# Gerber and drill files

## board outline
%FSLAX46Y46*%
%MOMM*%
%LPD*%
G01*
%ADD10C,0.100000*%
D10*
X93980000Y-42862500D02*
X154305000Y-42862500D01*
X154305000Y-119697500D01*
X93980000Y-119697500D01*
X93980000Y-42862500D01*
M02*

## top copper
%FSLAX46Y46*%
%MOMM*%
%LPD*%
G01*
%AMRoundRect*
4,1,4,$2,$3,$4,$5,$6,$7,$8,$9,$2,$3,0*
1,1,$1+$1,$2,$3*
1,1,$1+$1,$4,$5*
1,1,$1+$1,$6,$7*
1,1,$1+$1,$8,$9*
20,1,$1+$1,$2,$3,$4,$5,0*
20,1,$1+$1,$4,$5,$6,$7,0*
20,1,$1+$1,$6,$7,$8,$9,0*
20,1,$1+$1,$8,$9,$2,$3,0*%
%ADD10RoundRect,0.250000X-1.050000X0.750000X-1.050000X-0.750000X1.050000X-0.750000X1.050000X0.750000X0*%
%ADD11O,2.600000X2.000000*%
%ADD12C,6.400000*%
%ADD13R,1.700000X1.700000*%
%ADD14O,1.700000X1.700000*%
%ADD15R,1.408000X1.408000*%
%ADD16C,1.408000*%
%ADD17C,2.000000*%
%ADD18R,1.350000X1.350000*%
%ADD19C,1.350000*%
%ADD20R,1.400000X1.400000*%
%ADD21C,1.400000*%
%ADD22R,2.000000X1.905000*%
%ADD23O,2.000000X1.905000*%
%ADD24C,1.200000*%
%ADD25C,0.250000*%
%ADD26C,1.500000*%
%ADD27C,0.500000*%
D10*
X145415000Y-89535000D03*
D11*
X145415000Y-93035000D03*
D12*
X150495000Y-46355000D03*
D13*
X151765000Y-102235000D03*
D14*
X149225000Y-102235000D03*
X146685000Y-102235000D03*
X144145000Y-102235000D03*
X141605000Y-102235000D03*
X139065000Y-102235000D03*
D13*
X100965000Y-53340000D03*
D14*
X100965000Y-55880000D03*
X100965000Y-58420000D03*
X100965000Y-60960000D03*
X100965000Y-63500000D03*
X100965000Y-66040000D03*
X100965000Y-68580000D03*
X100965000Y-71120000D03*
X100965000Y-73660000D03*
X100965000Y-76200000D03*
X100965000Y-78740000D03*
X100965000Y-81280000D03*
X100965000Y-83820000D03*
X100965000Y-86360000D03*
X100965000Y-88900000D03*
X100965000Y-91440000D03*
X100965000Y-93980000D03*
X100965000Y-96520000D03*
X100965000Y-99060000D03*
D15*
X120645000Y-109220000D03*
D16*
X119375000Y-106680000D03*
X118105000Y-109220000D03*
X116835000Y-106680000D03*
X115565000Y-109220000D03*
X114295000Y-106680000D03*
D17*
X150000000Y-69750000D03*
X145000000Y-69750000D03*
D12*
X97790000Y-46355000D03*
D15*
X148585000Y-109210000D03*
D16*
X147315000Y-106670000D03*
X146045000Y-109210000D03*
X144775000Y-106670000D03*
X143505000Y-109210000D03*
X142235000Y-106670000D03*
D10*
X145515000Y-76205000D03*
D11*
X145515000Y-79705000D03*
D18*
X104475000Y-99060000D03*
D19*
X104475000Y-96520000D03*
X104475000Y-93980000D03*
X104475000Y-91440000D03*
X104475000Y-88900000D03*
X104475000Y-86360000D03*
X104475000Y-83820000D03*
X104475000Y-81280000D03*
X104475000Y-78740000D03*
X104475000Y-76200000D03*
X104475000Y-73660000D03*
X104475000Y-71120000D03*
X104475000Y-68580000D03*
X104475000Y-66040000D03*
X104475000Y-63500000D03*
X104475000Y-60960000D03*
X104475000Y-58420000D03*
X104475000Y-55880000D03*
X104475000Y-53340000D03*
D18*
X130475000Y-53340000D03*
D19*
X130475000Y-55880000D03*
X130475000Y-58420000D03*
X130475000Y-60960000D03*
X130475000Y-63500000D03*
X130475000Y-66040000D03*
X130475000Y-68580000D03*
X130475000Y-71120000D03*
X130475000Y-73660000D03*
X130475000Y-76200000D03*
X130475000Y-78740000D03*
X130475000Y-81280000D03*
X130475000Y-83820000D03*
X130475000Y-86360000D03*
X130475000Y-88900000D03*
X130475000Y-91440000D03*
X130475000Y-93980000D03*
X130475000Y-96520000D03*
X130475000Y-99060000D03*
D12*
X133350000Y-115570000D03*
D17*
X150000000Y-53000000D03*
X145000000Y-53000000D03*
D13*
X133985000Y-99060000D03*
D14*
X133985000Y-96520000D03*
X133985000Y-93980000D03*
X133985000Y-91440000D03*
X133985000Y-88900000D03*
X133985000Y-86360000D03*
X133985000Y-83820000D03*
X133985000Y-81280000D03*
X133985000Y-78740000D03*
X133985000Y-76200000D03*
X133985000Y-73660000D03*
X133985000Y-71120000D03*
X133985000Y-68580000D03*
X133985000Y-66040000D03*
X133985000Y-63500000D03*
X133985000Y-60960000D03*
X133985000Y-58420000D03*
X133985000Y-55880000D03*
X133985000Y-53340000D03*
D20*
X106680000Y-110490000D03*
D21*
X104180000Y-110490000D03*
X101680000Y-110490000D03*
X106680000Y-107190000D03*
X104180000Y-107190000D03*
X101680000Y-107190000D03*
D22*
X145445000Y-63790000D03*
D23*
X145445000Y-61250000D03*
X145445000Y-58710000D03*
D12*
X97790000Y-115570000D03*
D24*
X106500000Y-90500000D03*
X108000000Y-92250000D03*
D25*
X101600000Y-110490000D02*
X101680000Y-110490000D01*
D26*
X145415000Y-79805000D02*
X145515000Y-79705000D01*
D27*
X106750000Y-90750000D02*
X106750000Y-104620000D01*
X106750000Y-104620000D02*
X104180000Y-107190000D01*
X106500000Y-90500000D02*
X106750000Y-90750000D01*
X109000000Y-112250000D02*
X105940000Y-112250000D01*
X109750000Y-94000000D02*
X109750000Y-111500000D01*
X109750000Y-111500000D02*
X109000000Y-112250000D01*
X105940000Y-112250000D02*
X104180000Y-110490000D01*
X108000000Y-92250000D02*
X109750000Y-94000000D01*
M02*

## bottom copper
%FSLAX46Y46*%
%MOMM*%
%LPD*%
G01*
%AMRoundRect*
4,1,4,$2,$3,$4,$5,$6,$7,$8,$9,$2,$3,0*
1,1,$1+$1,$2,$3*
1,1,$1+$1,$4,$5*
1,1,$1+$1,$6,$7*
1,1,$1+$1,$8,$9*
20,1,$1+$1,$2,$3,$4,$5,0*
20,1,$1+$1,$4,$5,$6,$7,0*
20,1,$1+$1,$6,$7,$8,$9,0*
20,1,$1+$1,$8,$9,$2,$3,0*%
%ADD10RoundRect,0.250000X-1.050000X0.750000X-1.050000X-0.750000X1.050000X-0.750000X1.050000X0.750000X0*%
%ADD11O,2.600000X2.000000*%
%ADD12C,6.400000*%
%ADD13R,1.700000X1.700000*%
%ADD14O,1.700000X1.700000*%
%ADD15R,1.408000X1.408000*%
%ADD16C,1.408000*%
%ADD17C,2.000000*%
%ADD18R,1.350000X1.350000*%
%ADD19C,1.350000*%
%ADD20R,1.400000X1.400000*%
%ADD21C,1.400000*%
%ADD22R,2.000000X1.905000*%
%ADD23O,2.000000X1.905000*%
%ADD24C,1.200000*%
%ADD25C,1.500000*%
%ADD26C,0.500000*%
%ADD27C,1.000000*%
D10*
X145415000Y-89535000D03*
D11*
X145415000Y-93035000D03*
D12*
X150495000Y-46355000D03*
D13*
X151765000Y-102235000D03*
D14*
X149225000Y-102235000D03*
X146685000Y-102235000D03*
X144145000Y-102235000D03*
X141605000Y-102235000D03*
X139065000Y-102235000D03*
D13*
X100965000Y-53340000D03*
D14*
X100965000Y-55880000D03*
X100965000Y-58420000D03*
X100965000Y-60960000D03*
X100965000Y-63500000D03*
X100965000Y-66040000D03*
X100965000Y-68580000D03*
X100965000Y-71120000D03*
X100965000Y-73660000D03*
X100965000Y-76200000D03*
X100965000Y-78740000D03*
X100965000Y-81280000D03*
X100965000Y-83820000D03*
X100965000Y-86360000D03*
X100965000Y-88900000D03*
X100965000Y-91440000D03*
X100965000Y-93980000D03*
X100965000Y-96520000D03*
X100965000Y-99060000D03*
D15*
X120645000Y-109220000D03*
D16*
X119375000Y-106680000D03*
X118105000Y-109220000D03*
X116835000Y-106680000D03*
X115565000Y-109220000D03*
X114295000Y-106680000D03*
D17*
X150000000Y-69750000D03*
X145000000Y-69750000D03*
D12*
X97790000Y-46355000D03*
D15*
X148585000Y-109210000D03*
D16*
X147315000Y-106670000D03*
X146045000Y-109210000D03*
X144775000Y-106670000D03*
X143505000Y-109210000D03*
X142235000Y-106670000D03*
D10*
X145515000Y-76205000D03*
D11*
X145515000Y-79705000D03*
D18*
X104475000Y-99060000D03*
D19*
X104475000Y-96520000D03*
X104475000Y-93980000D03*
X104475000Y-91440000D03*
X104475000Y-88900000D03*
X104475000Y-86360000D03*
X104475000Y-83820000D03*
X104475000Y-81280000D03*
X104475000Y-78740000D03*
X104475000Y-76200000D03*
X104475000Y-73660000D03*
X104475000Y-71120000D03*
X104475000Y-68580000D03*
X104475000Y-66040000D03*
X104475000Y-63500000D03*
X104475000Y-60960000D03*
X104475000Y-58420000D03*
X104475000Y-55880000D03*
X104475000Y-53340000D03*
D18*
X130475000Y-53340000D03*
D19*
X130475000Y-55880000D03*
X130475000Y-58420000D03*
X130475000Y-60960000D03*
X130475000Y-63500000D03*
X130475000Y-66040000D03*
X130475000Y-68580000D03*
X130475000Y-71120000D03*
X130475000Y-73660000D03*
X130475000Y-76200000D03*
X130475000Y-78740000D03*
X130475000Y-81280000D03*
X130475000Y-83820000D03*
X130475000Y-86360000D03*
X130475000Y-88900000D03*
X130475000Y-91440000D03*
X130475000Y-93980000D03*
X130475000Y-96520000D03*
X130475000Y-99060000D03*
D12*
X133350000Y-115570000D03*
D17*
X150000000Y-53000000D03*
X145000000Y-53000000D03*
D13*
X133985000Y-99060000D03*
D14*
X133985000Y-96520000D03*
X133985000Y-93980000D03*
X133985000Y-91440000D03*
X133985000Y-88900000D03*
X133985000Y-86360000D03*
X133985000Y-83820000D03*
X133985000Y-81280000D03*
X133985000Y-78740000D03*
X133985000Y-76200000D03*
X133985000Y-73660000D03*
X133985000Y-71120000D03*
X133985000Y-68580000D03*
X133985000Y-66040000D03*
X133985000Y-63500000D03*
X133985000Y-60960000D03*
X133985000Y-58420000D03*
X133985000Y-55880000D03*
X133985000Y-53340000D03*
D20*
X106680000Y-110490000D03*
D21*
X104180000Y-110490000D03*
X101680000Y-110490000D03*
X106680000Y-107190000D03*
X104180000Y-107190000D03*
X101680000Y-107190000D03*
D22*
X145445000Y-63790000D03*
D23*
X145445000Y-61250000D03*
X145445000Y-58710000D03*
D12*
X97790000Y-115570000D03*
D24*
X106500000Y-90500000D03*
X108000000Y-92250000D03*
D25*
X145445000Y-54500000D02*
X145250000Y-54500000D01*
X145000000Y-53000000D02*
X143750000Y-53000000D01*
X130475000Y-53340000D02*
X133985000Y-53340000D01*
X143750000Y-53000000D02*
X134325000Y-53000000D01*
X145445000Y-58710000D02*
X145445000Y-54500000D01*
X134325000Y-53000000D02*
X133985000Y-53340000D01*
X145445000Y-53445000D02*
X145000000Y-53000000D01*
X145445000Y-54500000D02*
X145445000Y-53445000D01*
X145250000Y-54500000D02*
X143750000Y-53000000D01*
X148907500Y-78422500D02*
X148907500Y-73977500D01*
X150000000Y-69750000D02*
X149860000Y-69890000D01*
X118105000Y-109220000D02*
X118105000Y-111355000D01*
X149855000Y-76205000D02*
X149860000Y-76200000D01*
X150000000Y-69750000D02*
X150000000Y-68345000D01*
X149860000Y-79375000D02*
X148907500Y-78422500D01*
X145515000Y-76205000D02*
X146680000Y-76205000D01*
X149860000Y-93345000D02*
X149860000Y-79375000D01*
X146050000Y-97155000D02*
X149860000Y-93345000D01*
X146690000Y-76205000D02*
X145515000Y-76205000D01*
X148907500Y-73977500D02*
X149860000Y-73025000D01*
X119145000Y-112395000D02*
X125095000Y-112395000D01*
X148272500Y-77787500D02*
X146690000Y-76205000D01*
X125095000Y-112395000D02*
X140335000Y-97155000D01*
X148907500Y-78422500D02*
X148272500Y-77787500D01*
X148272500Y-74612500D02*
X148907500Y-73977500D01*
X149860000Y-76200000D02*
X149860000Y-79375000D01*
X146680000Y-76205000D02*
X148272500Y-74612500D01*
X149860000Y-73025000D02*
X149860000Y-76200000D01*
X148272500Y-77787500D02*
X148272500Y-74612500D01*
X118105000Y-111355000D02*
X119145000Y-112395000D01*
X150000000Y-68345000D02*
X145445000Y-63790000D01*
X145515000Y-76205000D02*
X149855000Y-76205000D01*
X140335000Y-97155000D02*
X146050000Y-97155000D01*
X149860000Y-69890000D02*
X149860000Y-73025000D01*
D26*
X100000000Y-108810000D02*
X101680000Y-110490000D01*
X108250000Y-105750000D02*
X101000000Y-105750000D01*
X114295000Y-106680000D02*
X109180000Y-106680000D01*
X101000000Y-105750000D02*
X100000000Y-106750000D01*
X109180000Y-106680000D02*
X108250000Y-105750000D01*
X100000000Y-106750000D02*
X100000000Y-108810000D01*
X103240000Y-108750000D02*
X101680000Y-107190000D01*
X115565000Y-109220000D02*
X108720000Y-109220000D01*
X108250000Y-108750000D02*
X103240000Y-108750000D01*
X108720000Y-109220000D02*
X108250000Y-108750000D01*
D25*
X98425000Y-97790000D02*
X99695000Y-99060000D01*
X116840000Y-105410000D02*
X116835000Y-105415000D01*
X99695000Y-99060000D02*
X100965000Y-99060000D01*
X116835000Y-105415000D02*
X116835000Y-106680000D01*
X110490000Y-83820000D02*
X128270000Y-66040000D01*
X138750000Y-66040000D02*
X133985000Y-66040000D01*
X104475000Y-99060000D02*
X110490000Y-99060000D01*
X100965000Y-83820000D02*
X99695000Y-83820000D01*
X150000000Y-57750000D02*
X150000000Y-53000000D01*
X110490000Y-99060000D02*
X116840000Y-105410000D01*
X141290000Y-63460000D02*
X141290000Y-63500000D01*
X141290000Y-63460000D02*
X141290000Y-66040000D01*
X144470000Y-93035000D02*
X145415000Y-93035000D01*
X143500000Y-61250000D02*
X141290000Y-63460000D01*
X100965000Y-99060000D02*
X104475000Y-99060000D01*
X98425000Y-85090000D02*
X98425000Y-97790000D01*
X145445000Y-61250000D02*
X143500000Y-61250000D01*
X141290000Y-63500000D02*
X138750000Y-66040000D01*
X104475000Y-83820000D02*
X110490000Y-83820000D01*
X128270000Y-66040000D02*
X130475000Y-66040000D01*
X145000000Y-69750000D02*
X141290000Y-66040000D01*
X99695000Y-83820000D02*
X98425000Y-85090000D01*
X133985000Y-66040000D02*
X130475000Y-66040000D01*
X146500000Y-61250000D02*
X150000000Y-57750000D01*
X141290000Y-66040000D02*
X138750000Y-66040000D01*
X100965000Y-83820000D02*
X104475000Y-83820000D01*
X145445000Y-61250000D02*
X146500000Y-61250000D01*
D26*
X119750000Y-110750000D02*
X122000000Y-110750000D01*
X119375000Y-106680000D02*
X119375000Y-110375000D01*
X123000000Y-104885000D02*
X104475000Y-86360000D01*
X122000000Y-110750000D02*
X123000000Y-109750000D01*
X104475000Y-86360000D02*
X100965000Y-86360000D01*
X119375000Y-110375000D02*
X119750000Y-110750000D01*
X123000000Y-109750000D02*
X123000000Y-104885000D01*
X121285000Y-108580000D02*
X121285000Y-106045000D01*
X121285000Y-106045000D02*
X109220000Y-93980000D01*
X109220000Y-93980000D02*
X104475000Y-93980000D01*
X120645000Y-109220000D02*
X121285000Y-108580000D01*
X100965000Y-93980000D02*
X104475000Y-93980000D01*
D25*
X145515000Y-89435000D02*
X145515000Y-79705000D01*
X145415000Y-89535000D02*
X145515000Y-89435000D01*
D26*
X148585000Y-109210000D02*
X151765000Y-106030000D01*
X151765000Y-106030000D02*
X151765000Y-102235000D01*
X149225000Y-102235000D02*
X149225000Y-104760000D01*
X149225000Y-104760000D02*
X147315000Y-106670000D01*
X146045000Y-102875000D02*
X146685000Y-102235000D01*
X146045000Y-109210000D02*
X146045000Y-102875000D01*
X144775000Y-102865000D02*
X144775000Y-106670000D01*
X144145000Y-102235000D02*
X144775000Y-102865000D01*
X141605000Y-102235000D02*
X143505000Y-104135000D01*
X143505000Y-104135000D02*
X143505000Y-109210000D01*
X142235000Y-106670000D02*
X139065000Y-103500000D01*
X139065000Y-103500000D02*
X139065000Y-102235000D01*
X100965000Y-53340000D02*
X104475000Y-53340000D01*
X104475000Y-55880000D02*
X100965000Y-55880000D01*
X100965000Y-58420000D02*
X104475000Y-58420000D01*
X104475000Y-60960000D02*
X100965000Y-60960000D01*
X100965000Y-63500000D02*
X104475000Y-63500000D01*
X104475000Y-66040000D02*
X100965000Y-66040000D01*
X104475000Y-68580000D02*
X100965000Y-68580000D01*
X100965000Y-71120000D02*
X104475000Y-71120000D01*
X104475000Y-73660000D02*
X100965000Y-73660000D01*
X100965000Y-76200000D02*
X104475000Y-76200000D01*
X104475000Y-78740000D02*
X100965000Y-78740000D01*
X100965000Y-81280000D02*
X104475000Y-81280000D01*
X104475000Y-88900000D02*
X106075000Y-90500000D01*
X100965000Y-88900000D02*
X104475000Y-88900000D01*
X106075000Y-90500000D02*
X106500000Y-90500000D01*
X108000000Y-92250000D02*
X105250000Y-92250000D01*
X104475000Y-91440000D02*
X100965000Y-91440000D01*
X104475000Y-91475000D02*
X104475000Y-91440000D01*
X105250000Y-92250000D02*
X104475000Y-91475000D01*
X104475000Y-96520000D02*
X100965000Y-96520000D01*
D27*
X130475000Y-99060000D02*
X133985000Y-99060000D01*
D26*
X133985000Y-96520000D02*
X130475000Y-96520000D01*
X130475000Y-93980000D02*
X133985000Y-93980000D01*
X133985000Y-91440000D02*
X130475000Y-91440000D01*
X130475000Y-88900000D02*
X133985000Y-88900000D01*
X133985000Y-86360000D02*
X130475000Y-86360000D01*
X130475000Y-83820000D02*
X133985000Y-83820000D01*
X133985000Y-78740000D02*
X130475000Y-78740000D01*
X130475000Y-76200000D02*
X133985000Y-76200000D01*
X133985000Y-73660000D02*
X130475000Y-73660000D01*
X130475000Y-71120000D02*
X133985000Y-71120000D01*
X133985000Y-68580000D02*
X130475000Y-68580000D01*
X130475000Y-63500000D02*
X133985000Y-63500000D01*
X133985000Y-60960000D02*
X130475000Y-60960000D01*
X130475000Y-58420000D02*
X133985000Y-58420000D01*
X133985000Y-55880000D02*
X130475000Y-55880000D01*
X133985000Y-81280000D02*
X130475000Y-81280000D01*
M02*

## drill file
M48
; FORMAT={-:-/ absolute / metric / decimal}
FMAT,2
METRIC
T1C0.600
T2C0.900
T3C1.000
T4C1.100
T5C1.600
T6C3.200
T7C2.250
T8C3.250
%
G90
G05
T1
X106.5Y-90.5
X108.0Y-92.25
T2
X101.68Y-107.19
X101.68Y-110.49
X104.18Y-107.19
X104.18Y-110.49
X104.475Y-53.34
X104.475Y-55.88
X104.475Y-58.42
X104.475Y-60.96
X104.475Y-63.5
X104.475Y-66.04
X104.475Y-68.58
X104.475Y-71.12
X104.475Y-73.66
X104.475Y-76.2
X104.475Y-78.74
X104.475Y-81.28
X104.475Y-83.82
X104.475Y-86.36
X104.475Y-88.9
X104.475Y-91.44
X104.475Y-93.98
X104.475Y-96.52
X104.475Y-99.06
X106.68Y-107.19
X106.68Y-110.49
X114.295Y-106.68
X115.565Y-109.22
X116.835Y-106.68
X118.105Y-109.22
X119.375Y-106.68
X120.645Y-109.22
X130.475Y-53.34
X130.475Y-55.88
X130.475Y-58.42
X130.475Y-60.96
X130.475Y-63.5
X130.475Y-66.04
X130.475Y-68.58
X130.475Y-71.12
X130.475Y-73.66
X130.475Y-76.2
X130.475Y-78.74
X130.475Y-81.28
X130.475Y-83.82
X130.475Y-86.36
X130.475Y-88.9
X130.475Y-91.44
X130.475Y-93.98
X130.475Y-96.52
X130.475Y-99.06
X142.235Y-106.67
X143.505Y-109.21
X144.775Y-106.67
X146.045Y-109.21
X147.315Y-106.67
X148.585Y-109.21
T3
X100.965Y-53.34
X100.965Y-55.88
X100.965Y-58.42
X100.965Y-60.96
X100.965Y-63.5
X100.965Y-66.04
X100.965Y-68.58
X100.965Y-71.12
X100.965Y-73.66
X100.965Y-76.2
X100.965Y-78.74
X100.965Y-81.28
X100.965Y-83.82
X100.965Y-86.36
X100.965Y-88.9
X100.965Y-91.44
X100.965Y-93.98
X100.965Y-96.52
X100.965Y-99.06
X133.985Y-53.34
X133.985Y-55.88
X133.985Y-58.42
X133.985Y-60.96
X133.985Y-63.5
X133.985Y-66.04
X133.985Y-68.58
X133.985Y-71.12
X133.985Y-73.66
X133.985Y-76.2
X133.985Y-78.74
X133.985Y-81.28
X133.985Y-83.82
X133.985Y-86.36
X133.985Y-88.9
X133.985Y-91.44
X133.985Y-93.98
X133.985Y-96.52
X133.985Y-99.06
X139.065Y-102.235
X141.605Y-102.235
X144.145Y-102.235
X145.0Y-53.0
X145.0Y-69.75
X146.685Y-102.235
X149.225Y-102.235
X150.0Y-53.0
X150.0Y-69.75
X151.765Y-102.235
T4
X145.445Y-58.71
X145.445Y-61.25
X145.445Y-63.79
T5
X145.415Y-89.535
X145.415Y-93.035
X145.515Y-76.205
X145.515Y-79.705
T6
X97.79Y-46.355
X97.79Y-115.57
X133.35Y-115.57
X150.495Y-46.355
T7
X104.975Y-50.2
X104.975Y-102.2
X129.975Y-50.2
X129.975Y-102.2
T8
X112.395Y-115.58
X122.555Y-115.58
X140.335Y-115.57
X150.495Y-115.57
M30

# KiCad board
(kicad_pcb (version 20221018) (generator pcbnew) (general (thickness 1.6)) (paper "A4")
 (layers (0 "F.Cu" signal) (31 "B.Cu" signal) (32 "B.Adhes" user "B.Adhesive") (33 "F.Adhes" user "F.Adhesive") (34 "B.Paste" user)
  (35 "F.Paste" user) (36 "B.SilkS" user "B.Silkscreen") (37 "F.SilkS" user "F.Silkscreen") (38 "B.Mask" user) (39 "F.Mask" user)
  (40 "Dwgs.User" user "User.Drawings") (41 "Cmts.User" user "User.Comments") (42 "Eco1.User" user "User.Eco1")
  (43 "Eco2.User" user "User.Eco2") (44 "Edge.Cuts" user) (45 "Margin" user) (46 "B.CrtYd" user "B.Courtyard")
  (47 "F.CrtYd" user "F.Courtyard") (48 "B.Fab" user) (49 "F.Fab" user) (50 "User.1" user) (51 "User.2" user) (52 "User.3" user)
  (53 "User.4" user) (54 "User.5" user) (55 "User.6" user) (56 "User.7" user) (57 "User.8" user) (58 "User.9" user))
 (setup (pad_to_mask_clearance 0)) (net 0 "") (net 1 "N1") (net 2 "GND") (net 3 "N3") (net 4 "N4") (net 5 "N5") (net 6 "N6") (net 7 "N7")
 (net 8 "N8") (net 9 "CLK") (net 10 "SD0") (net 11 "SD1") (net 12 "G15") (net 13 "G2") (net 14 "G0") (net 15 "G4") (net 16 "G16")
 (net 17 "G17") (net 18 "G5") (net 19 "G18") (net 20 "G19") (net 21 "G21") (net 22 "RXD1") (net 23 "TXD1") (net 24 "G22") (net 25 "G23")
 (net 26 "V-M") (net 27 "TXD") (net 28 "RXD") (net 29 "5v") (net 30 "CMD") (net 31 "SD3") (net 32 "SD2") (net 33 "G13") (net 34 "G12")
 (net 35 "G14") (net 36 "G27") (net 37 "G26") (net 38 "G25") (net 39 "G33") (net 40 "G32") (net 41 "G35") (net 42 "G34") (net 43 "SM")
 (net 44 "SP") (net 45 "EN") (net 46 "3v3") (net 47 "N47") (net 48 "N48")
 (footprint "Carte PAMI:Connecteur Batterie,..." (layer "F.Cu") (at 145.415 89.535 -90)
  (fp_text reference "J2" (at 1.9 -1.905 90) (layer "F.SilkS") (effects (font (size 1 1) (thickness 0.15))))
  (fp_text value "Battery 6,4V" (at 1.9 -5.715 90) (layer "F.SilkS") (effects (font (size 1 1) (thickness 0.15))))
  (pad "1" thru_hole roundrect (at 0 0 270) (size 2 2.6) (drill 1.6) (layers "*.Cu" "*.Mask") (roundrect_rratio 0.125) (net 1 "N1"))
  (pad "2" thru_hole oval (at 3.5 0 270) (size 2 2.6) (drill 1.6) (layers "*.Cu" "*.Mask") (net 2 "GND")))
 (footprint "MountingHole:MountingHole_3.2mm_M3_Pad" (layer "F.Cu") (at 150.495 46.355)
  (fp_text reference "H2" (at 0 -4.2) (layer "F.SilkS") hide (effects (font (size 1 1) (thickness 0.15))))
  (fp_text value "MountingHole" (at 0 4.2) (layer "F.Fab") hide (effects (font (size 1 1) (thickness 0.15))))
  (pad "1" thru_hole circle (at 0 0) (size 6.4 6.4) (drill 3.2) (layers "*.Cu" "*.Mask")))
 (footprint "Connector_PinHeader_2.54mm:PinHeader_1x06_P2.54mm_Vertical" (layer "F.Cu") (at 151.765 102.235 -90)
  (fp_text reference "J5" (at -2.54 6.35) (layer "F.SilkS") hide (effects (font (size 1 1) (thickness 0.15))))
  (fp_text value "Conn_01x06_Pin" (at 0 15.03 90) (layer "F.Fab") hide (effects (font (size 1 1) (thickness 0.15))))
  (pad "1" thru_hole rect (at 0 0 270) (size 1.7 1.7) (drill 1) (layers "*.Cu" "*.Mask") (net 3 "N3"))
  (pad "2" thru_hole oval (at 0 2.54 270) (size 1.7 1.7) (drill 1) (layers "*.Cu" "*.Mask") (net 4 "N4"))
  (pad "3" thru_hole oval (at 0 5.08 270) (size 1.7 1.7) (drill 1) (layers "*.Cu" "*.Mask") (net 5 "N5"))
  (pad "4" thru_hole oval (at 0 7.62 270) (size 1.7 1.7) (drill 1) (layers "*.Cu" "*.Mask") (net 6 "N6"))
  (pad "5" thru_hole oval (at 0 10.16 270) (size 1.7 1.7) (drill 1) (layers "*.Cu" "*.Mask") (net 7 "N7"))
  (pad "6" thru_hole oval (at 0 12.7 270) (size 1.7 1.7) (drill 1) (layers "*.Cu" "*.Mask") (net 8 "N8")))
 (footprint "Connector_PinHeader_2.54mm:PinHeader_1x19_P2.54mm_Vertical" (layer "F.Cu") (at 100.965 53.34)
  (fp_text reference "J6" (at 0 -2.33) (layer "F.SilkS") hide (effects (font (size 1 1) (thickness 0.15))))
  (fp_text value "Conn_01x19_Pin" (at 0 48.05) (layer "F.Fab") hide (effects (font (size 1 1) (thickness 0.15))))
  (pad "1" thru_hole rect (at 0 0) (size 1.7 1.7) (drill 1) (layers "*.Cu" "*.Mask") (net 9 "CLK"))
  (pad "2" thru_hole oval (at 0 2.54) (size 1.7 1.7) (drill 1) (layers "*.Cu" "*.Mask") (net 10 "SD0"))
  (pad "3" thru_hole oval (at 0 5.08) (size 1.7 1.7) (drill 1) (layers "*.Cu" "*.Mask") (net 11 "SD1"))
  (pad "4" thru_hole oval (at 0 7.62) (size 1.7 1.7) (drill 1) (layers "*.Cu" "*.Mask") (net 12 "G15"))
  (pad "5" thru_hole oval (at 0 10.16) (size 1.7 1.7) (drill 1) (layers "*.Cu" "*.Mask") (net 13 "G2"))
  (pad "6" thru_hole oval (at 0 12.7) (size 1.7 1.7) (drill 1) (layers "*.Cu" "*.Mask") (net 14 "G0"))
  (pad "7" thru_hole oval (at 0 15.24) (size 1.7 1.7) (drill 1) (layers "*.Cu" "*.Mask") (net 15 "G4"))
  (pad "8" thru_hole oval (at 0 17.78) (size 1.7 1.7) (drill 1) (layers "*.Cu" "*.Mask") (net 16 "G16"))
  (pad "9" thru_hole oval (at 0 20.32) (size 1.7 1.7) (drill 1) (layers "*.Cu" "*.Mask") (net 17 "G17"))
  (pad "10" thru_hole oval (at 0 22.86) (size 1.7 1.7) (drill 1) (layers "*.Cu" "*.Mask") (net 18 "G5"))
  (pad "11" thru_hole oval (at 0 25.4) (size 1.7 1.7) (drill 1) (layers "*.Cu" "*.Mask") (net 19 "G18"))
  (pad "12" thru_hole oval (at 0 27.94) (size 1.7 1.7) (drill 1) (layers "*.Cu" "*.Mask") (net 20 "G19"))
  (pad "13" thru_hole oval (at 0 30.48) (size 1.7 1.7) (drill 1) (layers "*.Cu" "*.Mask") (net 2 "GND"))
  (pad "14" thru_hole oval (at 0 33.02) (size 1.7 1.7) (drill 1) (layers "*.Cu" "*.Mask") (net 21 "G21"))
  (pad "15" thru_hole oval (at 0 35.56) (size 1.7 1.7) (drill 1) (layers "*.Cu" "*.Mask") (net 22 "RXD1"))
  (pad "16" thru_hole oval (at 0 38.1) (size 1.7 1.7) (drill 1) (layers "*.Cu" "*.Mask") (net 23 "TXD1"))
  (pad "17" thru_hole oval (at 0 40.64) (size 1.7 1.7) (drill 1) (layers "*.Cu" "*.Mask") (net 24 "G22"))
  (pad "18" thru_hole oval (at 0 43.18) (size 1.7 1.7) (drill 1) (layers "*.Cu" "*.Mask") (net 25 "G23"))
  (pad "19" thru_hole oval (at 0 45.72) (size 1.7 1.7) (drill 1) (layers "*.Cu" "*.Mask") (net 2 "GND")))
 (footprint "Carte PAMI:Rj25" (layer "F.Cu") (at 117.475 109.22 -90)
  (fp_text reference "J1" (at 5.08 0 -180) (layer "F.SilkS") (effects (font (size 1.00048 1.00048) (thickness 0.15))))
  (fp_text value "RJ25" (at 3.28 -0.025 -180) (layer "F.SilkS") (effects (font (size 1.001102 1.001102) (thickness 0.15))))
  (pad "" np_thru_hole circle (at 6.36 -5.08 270) (size 3.25 3.25) (drill 3.25) (layers "*.Cu" "*.Mask"))
  (pad "" np_thru_hole circle (at 6.36 5.08 270) (size 3.25 3.25) (drill 3.25) (layers "*.Cu" "*.Mask"))
  (pad "1" thru_hole rect (at 0 -3.17 270) (size 1.408 1.408) (drill 0.9) (layers "*.Cu" "*.Mask") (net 24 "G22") (solder_mask_margin 0.102))
  (pad "2" thru_hole circle (at -2.54 -1.9 270) (size 1.408 1.408) (drill 0.9) (layers "*.Cu" "*.Mask") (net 21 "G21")
   (solder_mask_margin 0.102))
  (pad "3" thru_hole circle (at 0 -0.63 270) (size 1.408 1.408) (drill 0.9) (layers "*.Cu" "*.Mask") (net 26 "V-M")
   (solder_mask_margin 0.102))
  (pad "4" thru_hole circle (at -2.54 0.64 270) (size 1.408 1.408) (drill 0.9) (layers "*.Cu" "*.Mask") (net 2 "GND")
   (solder_mask_margin 0.102))
  (pad "5" thru_hole circle (at 0 1.91 270) (size 1.408 1.408) (drill 0.9) (layers "*.Cu" "*.Mask") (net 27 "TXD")
   (solder_mask_margin 0.102))
  (pad "6" thru_hole circle (at -2.54 3.18 270) (size 1.408 1.408) (drill 0.9) (layers "*.Cu" "*.Mask") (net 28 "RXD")
   (solder_mask_margin 0.102)))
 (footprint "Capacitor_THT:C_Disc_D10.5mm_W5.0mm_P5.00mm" (layer "F.Cu") (at 150 69.75 180)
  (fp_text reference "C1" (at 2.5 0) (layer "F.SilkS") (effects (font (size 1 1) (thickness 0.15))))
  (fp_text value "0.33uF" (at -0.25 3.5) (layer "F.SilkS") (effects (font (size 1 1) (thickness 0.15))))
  (pad "1" thru_hole circle (at 0 0 180) (size 2 2) (drill 1) (layers "*.Cu" "*.Mask") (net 26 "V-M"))
  (pad "2" thru_hole circle (at 5 0 180) (size 2 2) (drill 1) (layers "*.Cu" "*.Mask") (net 2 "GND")))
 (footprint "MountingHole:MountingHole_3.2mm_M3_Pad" (layer "F.Cu") (at 97.79 46.355)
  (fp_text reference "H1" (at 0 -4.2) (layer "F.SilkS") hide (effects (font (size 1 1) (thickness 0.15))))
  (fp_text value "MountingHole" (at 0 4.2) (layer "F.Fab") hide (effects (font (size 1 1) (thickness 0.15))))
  (pad "1" thru_hole circle (at 0 0) (size 6.4 6.4) (drill 3.2) (layers "*.Cu" "*.Mask")))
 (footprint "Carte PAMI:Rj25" (layer "F.Cu") (at 145.415 109.21 -90)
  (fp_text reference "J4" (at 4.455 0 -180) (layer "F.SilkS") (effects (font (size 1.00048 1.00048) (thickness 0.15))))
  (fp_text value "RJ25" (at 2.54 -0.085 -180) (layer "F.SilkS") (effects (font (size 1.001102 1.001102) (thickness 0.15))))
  (pad "" np_thru_hole circle (at 6.36 -5.08 270) (size 3.25 3.25) (drill 3.25) (layers "*.Cu" "*.Mask"))
  (pad "" np_thru_hole circle (at 6.36 5.08 270) (size 3.25 3.25) (drill 3.25) (layers "*.Cu" "*.Mask"))
  (pad "1" thru_hole rect (at 0 -3.17 270) (size 1.408 1.408) (drill 0.9) (layers "*.Cu" "*.Mask") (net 3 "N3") (solder_mask_margin 0.102))
  (pad "2" thru_hole circle (at -2.54 -1.9 270) (size 1.408 1.408) (drill 0.9) (layers "*.Cu" "*.Mask") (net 4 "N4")
   (solder_mask_margin 0.102))
  (pad "3" thru_hole circle (at 0 -0.63 270) (size 1.408 1.408) (drill 0.9) (layers "*.Cu" "*.Mask") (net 5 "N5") (solder_mask_margin 0.102))
  (pad "4" thru_hole circle (at -2.54 0.64 270) (size 1.408 1.408) (drill 0.9) (layers "*.Cu" "*.Mask") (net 6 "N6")
   (solder_mask_margin 0.102))
  (pad "5" thru_hole circle (at 0 1.91 270) (size 1.408 1.408) (drill 0.9) (layers "*.Cu" "*.Mask") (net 7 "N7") (solder_mask_margin 0.102))
  (pad "6" thru_hole circle (at -2.54 3.18 270) (size 1.408 1.408) (drill 0.9) (layers "*.Cu" "*.Mask") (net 8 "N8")
   (solder_mask_margin 0.102)))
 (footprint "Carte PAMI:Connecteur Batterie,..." (layer "F.Cu") (at 145.515 76.205 -90)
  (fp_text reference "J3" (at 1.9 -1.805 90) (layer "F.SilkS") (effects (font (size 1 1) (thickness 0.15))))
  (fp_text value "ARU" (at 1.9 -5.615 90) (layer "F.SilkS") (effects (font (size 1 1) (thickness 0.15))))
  (pad "1" thru_hole roundrect (at 0 0 270) (size 2 2.6) (drill 1.6) (layers "*.Cu" "*.Mask") (roundrect_rratio 0.125) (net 26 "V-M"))
  (pad "2" thru_hole oval (at 3.5 0 270) (size 2 2.6) (drill 1.6) (layers "*.Cu" "*.Mask") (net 1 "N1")))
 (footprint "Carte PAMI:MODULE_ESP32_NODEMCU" (layer "F.Cu") (at 117.475 76.2 180)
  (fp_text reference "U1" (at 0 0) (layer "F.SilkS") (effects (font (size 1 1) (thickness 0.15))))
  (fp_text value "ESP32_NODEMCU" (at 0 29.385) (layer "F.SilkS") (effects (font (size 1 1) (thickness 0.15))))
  (pad "" np_thru_hole circle (at -12.5 -26 180) (size 2.25 2.25) (drill 2.25) (layers "*.Cu" "*.Mask"))
  (pad "" np_thru_hole circle (at -12.5 26 180) (size 2.25 2.25) (drill 2.25) (layers "*.Cu" "*.Mask"))
  (pad "" np_thru_hole circle (at 12.5 -26 180) (size 2.25 2.25) (drill 2.25) (layers "*.Cu" "*.Mask"))
  (pad "" np_thru_hole circle (at 12.5 26 180) (size 2.25 2.25) (drill 2.25) (layers "*.Cu" "*.Mask"))
  (pad "J4_1" thru_hole rect (at 13 -22.86 180) (size 1.35 1.35) (drill 0.9) (layers "*.Cu" "*.Mask") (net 2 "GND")
   (solder_mask_margin 0.102))
  (pad "J4_2" thru_hole circle (at 13 -20.32 180) (size 1.35 1.35) (drill 0.9) (layers "*.Cu" "*.Mask") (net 25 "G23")
   (solder_mask_margin 0.102))
  (pad "J4_3" thru_hole circle (at 13 -17.78 180) (size 1.35 1.35) (drill 0.9) (layers "*.Cu" "*.Mask") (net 24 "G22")
   (solder_mask_margin 0.102))
  (pad "J4_4" thru_hole circle (at 13 -15.24 180) (size 1.35 1.35) (drill 0.9) (layers "*.Cu" "*.Mask") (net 23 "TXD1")
   (solder_mask_margin 0.102))
  (pad "J4_5" thru_hole circle (at 13 -12.7 180) (size 1.35 1.35) (drill 0.9) (layers "*.Cu" "*.Mask") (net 22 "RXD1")
   (solder_mask_margin 0.102))
  (pad "J4_6" thru_hole circle (at 13 -10.16 180) (size 1.35 1.35) (drill 0.9) (layers "*.Cu" "*.Mask") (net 21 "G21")
   (solder_mask_margin 0.102))
  (pad "J4_7" thru_hole circle (at 13 -7.62 180) (size 1.35 1.35) (drill 0.9) (layers "*.Cu" "*.Mask") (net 2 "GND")
   (solder_mask_margin 0.102))
  (pad "J4_8" thru_hole circle (at 13 -5.08 180) (size 1.35 1.35) (drill 0.9) (layers "*.Cu" "*.Mask") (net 20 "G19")
   (solder_mask_margin 0.102))
  (pad "J4_9" thru_hole circle (at 13 -2.54 180) (size 1.35 1.35) (drill 0.9) (layers "*.Cu" "*.Mask") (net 19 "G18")
   (solder_mask_margin 0.102))
  (pad "J4_10" thru_hole circle (at 13 0 180) (size 1.35 1.35) (drill 0.9) (layers "*.Cu" "*.Mask") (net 18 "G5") (solder_mask_margin 0.102))
  (pad "J4_11" thru_hole circle (at 13 2.54 180) (size 1.35 1.35) (drill 0.9) (layers "*.Cu" "*.Mask") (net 17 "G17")
   (solder_mask_margin 0.102))
  (pad "J4_12" thru_hole circle (at 13 5.08 180) (size 1.35 1.35) (drill 0.9) (layers "*.Cu" "*.Mask") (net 16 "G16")
   (solder_mask_margin 0.102))
  (pad "J4_13" thru_hole circle (at 13 7.62 180) (size 1.35 1.35) (drill 0.9) (layers "*.Cu" "*.Mask") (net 15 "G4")
   (solder_mask_margin 0.102))
  (pad "J4_14" thru_hole circle (at 13 10.16 180) (size 1.35 1.35) (drill 0.9) (layers "*.Cu" "*.Mask") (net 14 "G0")
   (solder_mask_margin 0.102))
  (pad "J4_15" thru_hole circle (at 13 12.7 180) (size 1.35 1.35) (drill 0.9) (layers "*.Cu" "*.Mask") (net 13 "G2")
   (solder_mask_margin 0.102))
  (pad "J4_16" thru_hole circle (at 13 15.24 180) (size 1.35 1.35) (drill 0.9) (layers "*.Cu" "*.Mask") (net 12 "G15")
   (solder_mask_margin 0.102))
  (pad "J4_17" thru_hole circle (at 13 17.78 180) (size 1.35 1.35) (drill 0.9) (layers "*.Cu" "*.Mask") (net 11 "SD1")
   (solder_mask_margin 0.102))
  (pad "J4_18" thru_hole circle (at 13 20.32 180) (size 1.35 1.35) (drill 0.9) (layers "*.Cu" "*.Mask") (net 10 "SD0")
   (solder_mask_margin 0.102))
  (pad "J4_19" thru_hole circle (at 13 22.86 180) (size 1.35 1.35) (drill 0.9) (layers "*.Cu" "*.Mask") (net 9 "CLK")
   (solder_mask_margin 0.102))
  (pad "J5_1" thru_hole rect (at -13 22.86 180) (size 1.35 1.35) (drill 0.9) (layers "*.Cu" "*.Mask") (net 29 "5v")
   (solder_mask_margin 0.102))
  (pad "J5_2" thru_hole circle (at -13 20.32 180) (size 1.35 1.35) (drill 0.9) (layers "*.Cu" "*.Mask") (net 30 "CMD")
   (solder_mask_margin 0.102))
  (pad "J5_3" thru_hole circle (at -13 17.78 180) (size 1.35 1.35) (drill 0.9) (layers "*.Cu" "*.Mask") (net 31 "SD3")
   (solder_mask_margin 0.102))
  (pad "J5_4" thru_hole circle (at -13 15.24 180) (size 1.35 1.35) (drill 0.9) (layers "*.Cu" "*.Mask") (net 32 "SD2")
   (solder_mask_margin 0.102))
  (pad "J5_5" thru_hole circle (at -13 12.7 180) (size 1.35 1.35) (drill 0.9) (layers "*.Cu" "*.Mask") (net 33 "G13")
   (solder_mask_margin 0.102))
  (pad "J5_6" thru_hole circle (at -13 10.16 180) (size 1.35 1.35) (drill 0.9) (layers "*.Cu" "*.Mask") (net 2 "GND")
   (solder_mask_margin 0.102))
  (pad "J5_7" thru_hole circle (at -13 7.62 180) (size 1.35 1.35) (drill 0.9) (layers "*.Cu" "*.Mask") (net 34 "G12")
   (solder_mask_margin 0.102))
  (pad "J5_8" thru_hole circle (at -13 5.08 180) (size 1.35 1.35) (drill 0.9) (layers "*.Cu" "*.Mask") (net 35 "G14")
   (solder_mask_margin 0.102))
  (pad "J5_9" thru_hole circle (at -13 2.54 180) (size 1.35 1.35) (drill 0.9) (layers "*.Cu" "*.Mask") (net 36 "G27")
   (solder_mask_margin 0.102))
  (pad "J5_10" thru_hole circle (at -13 0 180) (size 1.35 1.35) (drill 0.9) (layers "*.Cu" "*.Mask") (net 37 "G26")
   (solder_mask_margin 0.102))
  (pad "J5_11" thru_hole circle (at -13 -2.54 180) (size 1.35 1.35) (drill 0.9) (layers "*.Cu" "*.Mask") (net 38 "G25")
   (solder_mask_margin 0.102))
  (pad "J5_12" thru_hole circle (at -13 -5.08 180) (size 1.35 1.35) (drill 0.9) (layers "*.Cu" "*.Mask") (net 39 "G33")
   (solder_mask_margin 0.102))
  (pad "J5_13" thru_hole circle (at -13 -7.62 180) (size 1.35 1.35) (drill 0.9) (layers "*.Cu" "*.Mask") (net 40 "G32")
   (solder_mask_margin 0.102))
  (pad "J5_14" thru_hole circle (at -13 -10.16 180) (size 1.35 1.35) (drill 0.9) (layers "*.Cu" "*.Mask") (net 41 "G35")
   (solder_mask_margin 0.102))
  (pad "J5_15" thru_hole circle (at -13 -12.7 180) (size 1.35 1.35) (drill 0.9) (layers "*.Cu" "*.Mask") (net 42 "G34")
   (solder_mask_margin 0.102))
  (pad "J5_16" thru_hole circle (at -13 -15.24 180) (size 1.35 1.35) (drill 0.9) (layers "*.Cu" "*.Mask") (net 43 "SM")
   (solder_mask_margin 0.102))
  (pad "J5_17" thru_hole circle (at -13 -17.78 180) (size 1.35 1.35) (drill 0.9) (layers "*.Cu" "*.Mask") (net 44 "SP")
   (solder_mask_margin 0.102))
  (pad "J5_18" thru_hole circle (at -13 -20.32 180) (size 1.35 1.35) (drill 0.9) (layers "*.Cu" "*.Mask") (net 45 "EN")
   (solder_mask_margin 0.102))
  (pad "J5_19" thru_hole circle (at -13 -22.86 180) (size 1.35 1.35) (drill 0.9) (layers "*.Cu" "*.Mask") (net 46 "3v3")
   (solder_mask_margin 0.102)))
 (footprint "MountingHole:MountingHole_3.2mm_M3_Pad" (layer "F.Cu") (at 133.35 115.57)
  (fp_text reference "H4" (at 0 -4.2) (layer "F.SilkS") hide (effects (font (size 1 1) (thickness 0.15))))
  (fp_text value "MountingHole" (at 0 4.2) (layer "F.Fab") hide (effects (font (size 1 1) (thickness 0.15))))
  (pad "1" thru_hole circle (at 0 0) (size 6.4 6.4) (drill 3.2) (layers "*.Cu" "*.Mask")))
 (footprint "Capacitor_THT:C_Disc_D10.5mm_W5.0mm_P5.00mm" (layer "F.Cu") (at 150 53 180)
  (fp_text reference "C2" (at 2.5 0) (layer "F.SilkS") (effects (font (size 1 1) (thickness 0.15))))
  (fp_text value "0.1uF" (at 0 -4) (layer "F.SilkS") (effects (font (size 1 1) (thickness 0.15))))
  (pad "1" thru_hole circle (at 0 0 180) (size 2 2) (drill 1) (layers "*.Cu" "*.Mask") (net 2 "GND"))
  (pad "2" thru_hole circle (at 5 0 180) (size 2 2) (drill 1) (layers "*.Cu" "*.Mask") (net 29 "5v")))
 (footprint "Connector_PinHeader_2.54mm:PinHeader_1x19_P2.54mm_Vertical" (layer "F.Cu") (at 133.985 99.06 180)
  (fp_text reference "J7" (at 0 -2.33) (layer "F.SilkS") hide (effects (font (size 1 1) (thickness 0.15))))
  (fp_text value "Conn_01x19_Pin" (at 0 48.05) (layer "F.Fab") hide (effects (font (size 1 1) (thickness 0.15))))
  (pad "1" thru_hole rect (at 0 0 180) (size 1.7 1.7) (drill 1) (layers "*.Cu" "*.Mask") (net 46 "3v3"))
  (pad "2" thru_hole oval (at 0 2.54 180) (size 1.7 1.7) (drill 1) (layers "*.Cu" "*.Mask") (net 45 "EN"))
  (pad "3" thru_hole oval (at 0 5.08 180) (size 1.7 1.7) (drill 1) (layers "*.Cu" "*.Mask") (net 44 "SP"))
  (pad "4" thru_hole oval (at 0 7.62 180) (size 1.7 1.7) (drill 1) (layers "*.Cu" "*.Mask") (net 43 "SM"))
  (pad "5" thru_hole oval (at 0 10.16 180) (size 1.7 1.7) (drill 1) (layers "*.Cu" "*.Mask") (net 42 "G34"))
  (pad "6" thru_hole oval (at 0 12.7 180) (size 1.7 1.7) (drill 1) (layers "*.Cu" "*.Mask") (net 41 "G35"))
  (pad "7" thru_hole oval (at 0 15.24 180) (size 1.7 1.7) (drill 1) (layers "*.Cu" "*.Mask") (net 40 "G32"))
  (pad "8" thru_hole oval (at 0 17.78 180) (size 1.7 1.7) (drill 1) (layers "*.Cu" "*.Mask") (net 39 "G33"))
  (pad "9" thru_hole oval (at 0 20.32 180) (size 1.7 1.7) (drill 1) (layers "*.Cu" "*.Mask") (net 38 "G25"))
  (pad "10" thru_hole oval (at 0 22.86 180) (size 1.7 1.7) (drill 1) (layers "*.Cu" "*.Mask") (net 37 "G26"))
  (pad "11" thru_hole oval (at 0 25.4 180) (size 1.7 1.7) (drill 1) (layers "*.Cu" "*.Mask") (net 36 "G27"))
  (pad "12" thru_hole oval (at 0 27.94 180) (size 1.7 1.7) (drill 1) (layers "*.Cu" "*.Mask") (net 35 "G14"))
  (pad "13" thru_hole oval (at 0 30.48 180) (size 1.7 1.7) (drill 1) (layers "*.Cu" "*.Mask") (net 34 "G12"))
  (pad "14" thru_hole oval (at 0 33.02 180) (size 1.7 1.7) (drill 1) (layers "*.Cu" "*.Mask") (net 2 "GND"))
  (pad "15" thru_hole oval (at 0 35.56 180) (size 1.7 1.7) (drill 1) (layers "*.Cu" "*.Mask") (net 33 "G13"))
  (pad "16" thru_hole oval (at 0 38.1 180) (size 1.7 1.7) (drill 1) (layers "*.Cu" "*.Mask") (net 32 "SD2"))
  (pad "17" thru_hole oval (at 0 40.64 180) (size 1.7 1.7) (drill 1) (layers "*.Cu" "*.Mask") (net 31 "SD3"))
  (pad "18" thru_hole oval (at 0 43.18 180) (size 1.7 1.7) (drill 1) (layers "*.Cu" "*.Mask") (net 30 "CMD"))
  (pad "19" thru_hole oval (at 0 45.72 180) (size 1.7 1.7) (drill 1) (layers "*.Cu" "*.Mask") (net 29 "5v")))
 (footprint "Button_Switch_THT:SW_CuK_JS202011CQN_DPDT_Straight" (layer "F.Cu") (at 106.68 110.49 180)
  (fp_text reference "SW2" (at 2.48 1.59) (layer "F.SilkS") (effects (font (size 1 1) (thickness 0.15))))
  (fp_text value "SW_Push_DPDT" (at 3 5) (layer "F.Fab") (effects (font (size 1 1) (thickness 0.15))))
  (pad "1" thru_hole rect (at 0 0 180) (size 1.4 1.4) (drill 0.9) (layers "*.Cu" "*.Mask") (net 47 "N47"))
  (pad "2" thru_hole circle (at 2.5 0 180) (size 1.4 1.4) (drill 0.9) (layers "*.Cu" "*.Mask") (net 23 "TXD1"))
  (pad "3" thru_hole circle (at 5 0 180) (size 1.4 1.4) (drill 0.9) (layers "*.Cu" "*.Mask") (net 28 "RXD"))
  (pad "4" thru_hole circle (at 0 3.3 180) (size 1.4 1.4) (drill 0.9) (layers "*.Cu" "*.Mask") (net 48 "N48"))
  (pad "5" thru_hole circle (at 2.5 3.3 180) (size 1.4 1.4) (drill 0.9) (layers "*.Cu" "*.Mask") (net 22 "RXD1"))
  (pad "6" thru_hole circle (at 5 3.3 180) (size 1.4 1.4) (drill 0.9) (layers "*.Cu" "*.Mask") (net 27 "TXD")))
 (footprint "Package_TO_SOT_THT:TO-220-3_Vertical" (layer "F.Cu") (at 145.445 63.79 90)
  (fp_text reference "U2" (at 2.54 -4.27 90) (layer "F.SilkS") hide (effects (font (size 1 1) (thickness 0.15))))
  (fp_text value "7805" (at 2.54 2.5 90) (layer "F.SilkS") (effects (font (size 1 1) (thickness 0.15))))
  (pad "1" thru_hole rect (at 0 0 90) (size 1.905 2) (drill 1.1) (layers "*.Cu" "*.Mask") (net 26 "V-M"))
  (pad "2" thru_hole oval (at 2.54 0 90) (size 1.905 2) (drill 1.1) (layers "*.Cu" "*.Mask") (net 2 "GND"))
  (pad "3" thru_hole oval (at 5.08 0 90) (size 1.905 2) (drill 1.1) (layers "*.Cu" "*.Mask") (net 29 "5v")))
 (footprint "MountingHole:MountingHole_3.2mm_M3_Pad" (layer "F.Cu") (at 97.79 115.57)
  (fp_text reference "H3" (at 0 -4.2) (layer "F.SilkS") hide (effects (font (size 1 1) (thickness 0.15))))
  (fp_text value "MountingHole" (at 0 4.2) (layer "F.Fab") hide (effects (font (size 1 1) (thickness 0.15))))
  (pad "1" thru_hole circle (at 0 0) (size 6.4 6.4) (drill 3.2) (layers "*.Cu" "*.Mask")))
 (gr_rect (start 93.98 42.8625) (end 154.305 119.6975) (stroke (width 0.1) (type default)) (fill none) (layer "Edge.Cuts"))
 (segment (start 145.445 54.5) (end 145.25 54.5) (width 1.5) (layer "B.Cu") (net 29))
 (segment (start 145 53) (end 143.75 53) (width 1.5) (layer "B.Cu") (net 29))
 (segment (start 130.475 53.34) (end 133.985 53.34) (width 1.5) (layer "B.Cu") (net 29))
 (segment (start 143.75 53) (end 134.325 53) (width 1.5) (layer "B.Cu") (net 29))
 (segment (start 145.445 58.71) (end 145.445 54.5) (width 1.5) (layer "B.Cu") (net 29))
 (segment (start 134.325 53) (end 133.985 53.34) (width 1.5) (layer "B.Cu") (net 29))
 (segment (start 145.445 53.445) (end 145 53) (width 1.5) (layer "B.Cu") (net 29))
 (segment (start 145.445 54.5) (end 145.445 53.445) (width 1.5) (layer "B.Cu") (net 29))
 (segment (start 145.25 54.5) (end 143.75 53) (width 1.5) (layer "B.Cu") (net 29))
 (segment (start 148.9075 78.4225) (end 148.9075 73.9775) (width 1.5) (layer "B.Cu") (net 26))
 (segment (start 150 69.75) (end 149.86 69.89) (width 1.5) (layer "B.Cu") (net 26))
 (segment (start 118.105 109.22) (end 118.105 111.355) (width 1.5) (layer "B.Cu") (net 26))
 (segment (start 149.855 76.205) (end 149.86 76.2) (width 1.5) (layer "B.Cu") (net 26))
 (segment (start 150 69.75) (end 150 68.345) (width 1.5) (layer "B.Cu") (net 26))
 (segment (start 149.86 79.375) (end 148.9075 78.4225) (width 1.5) (layer "B.Cu") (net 26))
 (segment (start 145.515 76.205) (end 146.68 76.205) (width 1.5) (layer "B.Cu") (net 26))
 (segment (start 149.86 93.345) (end 149.86 79.375) (width 1.5) (layer "B.Cu") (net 26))
 (segment (start 146.05 97.155) (end 149.86 93.345) (width 1.5) (layer "B.Cu") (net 26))
 (segment (start 146.69 76.205) (end 145.515 76.205) (width 1.5) (layer "B.Cu") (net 26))
 (segment (start 148.9075 73.9775) (end 149.86 73.025) (width 1.5) (layer "B.Cu") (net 26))
 (segment (start 119.145 112.395) (end 125.095 112.395) (width 1.5) (layer "B.Cu") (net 26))
 (segment (start 148.2725 77.7875) (end 146.69 76.205) (width 1.5) (layer "B.Cu") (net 26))
 (segment (start 125.095 112.395) (end 140.335 97.155) (width 1.5) (layer "B.Cu") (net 26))
 (segment (start 148.9075 78.4225) (end 148.2725 77.7875) (width 1.5) (layer "B.Cu") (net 26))
 (segment (start 148.2725 74.6125) (end 148.9075 73.9775) (width 1.5) (layer "B.Cu") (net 26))
 (segment (start 149.86 76.2) (end 149.86 79.375) (width 1.5) (layer "B.Cu") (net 26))
 (segment (start 146.68 76.205) (end 148.2725 74.6125) (width 1.5) (layer "B.Cu") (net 26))
 (segment (start 149.86 73.025) (end 149.86 76.2) (width 1.5) (layer "B.Cu") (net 26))
 (segment (start 148.2725 77.7875) (end 148.2725 74.6125) (width 1.5) (layer "B.Cu") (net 26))
 (segment (start 118.105 111.355) (end 119.145 112.395) (width 1.5) (layer "B.Cu") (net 26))
 (segment (start 150 68.345) (end 145.445 63.79) (width 1.5) (layer "B.Cu") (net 26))
 (segment (start 145.515 76.205) (end 149.855 76.205) (width 1.5) (layer "B.Cu") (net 26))
 (segment (start 140.335 97.155) (end 146.05 97.155) (width 1.5) (layer "B.Cu") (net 26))
 (segment (start 149.86 69.89) (end 149.86 73.025) (width 1.5) (layer "B.Cu") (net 26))
 (segment (start 101.6 110.49) (end 101.68 110.49) (width 0.25) (layer "F.Cu") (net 28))
 (segment (start 100 108.81) (end 101.68 110.49) (width 0.5) (layer "B.Cu") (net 28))
 (segment (start 108.25 105.75) (end 101 105.75) (width 0.5) (layer "B.Cu") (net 28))
 (segment (start 114.295 106.68) (end 109.18 106.68) (width 0.5) (layer "B.Cu") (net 28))
 (segment (start 101 105.75) (end 100 106.75) (width 0.5) (layer "B.Cu") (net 28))
 (segment (start 109.18 106.68) (end 108.25 105.75) (width 0.5) (layer "B.Cu") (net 28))
 (segment (start 100 106.75) (end 100 108.81) (width 0.5) (layer "B.Cu") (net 28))
 (segment (start 103.24 108.75) (end 101.68 107.19) (width 0.5) (layer "B.Cu") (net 27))
 (segment (start 115.565 109.22) (end 108.72 109.22) (width 0.5) (layer "B.Cu") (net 27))
 (segment (start 108.25 108.75) (end 103.24 108.75) (width 0.5) (layer "B.Cu") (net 27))
 (segment (start 108.72 109.22) (end 108.25 108.75) (width 0.5) (layer "B.Cu") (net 27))
 (segment (start 98.425 97.79) (end 99.695 99.06) (width 1.5) (layer "B.Cu") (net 2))
 (segment (start 116.84 105.41) (end 116.835 105.415) (width 1.5) (layer "B.Cu") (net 2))
 (segment (start 99.695 99.06) (end 100.965 99.06) (width 1.5) (layer "B.Cu") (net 2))
 (segment (start 116.835 105.415) (end 116.835 106.68) (width 1.5) (layer "B.Cu") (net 2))
 (segment (start 110.49 83.82) (end 128.27 66.04) (width 1.5) (layer "B.Cu") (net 2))
 (segment (start 138.75 66.04) (end 133.985 66.04) (width 1.5) (layer "B.Cu") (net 2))
 (segment (start 104.475 99.06) (end 110.49 99.06) (width 1.5) (layer "B.Cu") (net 2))
 (segment (start 100.965 83.82) (end 99.695 83.82) (width 1.5) (layer "B.Cu") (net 2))
 (segment (start 150 57.75) (end 150 53) (width 1.5) (layer "B.Cu") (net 2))
 (segment (start 110.49 99.06) (end 116.84 105.41) (width 1.5) (layer "B.Cu") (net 2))
 (segment (start 141.29 63.46) (end 141.29 63.5) (width 1.5) (layer "B.Cu") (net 2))
 (segment (start 141.29 63.46) (end 141.29 66.04) (width 1.5) (layer "B.Cu") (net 2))
 (segment (start 144.47 93.035) (end 145.415 93.035) (width 1.5) (layer "B.Cu") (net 2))
 (segment (start 143.5 61.25) (end 141.29 63.46) (width 1.5) (layer "B.Cu") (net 2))
 (segment (start 100.965 99.06) (end 104.475 99.06) (width 1.5) (layer "B.Cu") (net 2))
 (segment (start 98.425 85.09) (end 98.425 97.79) (width 1.5) (layer "B.Cu") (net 2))
 (segment (start 145.445 61.25) (end 143.5 61.25) (width 1.5) (layer "B.Cu") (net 2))
 (segment (start 141.29 63.5) (end 138.75 66.04) (width 1.5) (layer "B.Cu") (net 2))
 (segment (start 104.475 83.82) (end 110.49 83.82) (width 1.5) (layer "B.Cu") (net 2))
 (segment (start 128.27 66.04) (end 130.475 66.04) (width 1.5) (layer "B.Cu") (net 2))
 (segment (start 145 69.75) (end 141.29 66.04) (width 1.5) (layer "B.Cu") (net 2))
 (segment (start 99.695 83.82) (end 98.425 85.09) (width 1.5) (layer "B.Cu") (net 2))
 (segment (start 133.985 66.04) (end 130.475 66.04) (width 1.5) (layer "B.Cu") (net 2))
 (segment (start 146.5 61.25) (end 150 57.75) (width 1.5) (layer "B.Cu") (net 2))
 (segment (start 141.29 66.04) (end 138.75 66.04) (width 1.5) (layer "B.Cu") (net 2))
 (segment (start 100.965 83.82) (end 104.475 83.82) (width 1.5) (layer "B.Cu") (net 2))
 (segment (start 145.445 61.25) (end 146.5 61.25) (width 1.5) (layer "B.Cu") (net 2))
 (segment (start 119.75 110.75) (end 122 110.75) (width 0.5) (layer "B.Cu") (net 21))
 (segment (start 119.375 106.68) (end 119.375 110.375) (width 0.5) (layer "B.Cu") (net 21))
 (segment (start 123 104.885) (end 104.475 86.36) (width 0.5) (layer "B.Cu") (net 21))
 (segment (start 122 110.75) (end 123 109.75) (width 0.5) (layer "B.Cu") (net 21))
 (segment (start 104.475 86.36) (end 100.965 86.36) (width 0.5) (layer "B.Cu") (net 21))
 (segment (start 119.375 110.375) (end 119.75 110.75) (width 0.5) (layer "B.Cu") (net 21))
 (segment (start 123 109.75) (end 123 104.885) (width 0.5) (layer "B.Cu") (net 21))
 (segment (start 121.285 108.58) (end 121.285 106.045) (width 0.5) (layer "B.Cu") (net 24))
 (segment (start 121.285 106.045) (end 109.22 93.98) (width 0.5) (layer "B.Cu") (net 24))
 (segment (start 109.22 93.98) (end 104.475 93.98) (width 0.5) (layer "B.Cu") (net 24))
 (segment (start 120.645 109.22) (end 121.285 108.58) (width 0.5) (layer "B.Cu") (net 24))
 (segment (start 100.965 93.98) (end 104.475 93.98) (width 0.5) (layer "B.Cu") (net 24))
 (segment (start 145.415 79.805) (end 145.515 79.705) (width 1.5) (layer "F.Cu") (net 1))
 (segment (start 145.515 89.435) (end 145.515 79.705) (width 1.5) (layer "B.Cu") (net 1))
 (segment (start 145.415 89.535) (end 145.515 89.435) (width 1.5) (layer "B.Cu") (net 1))
 (segment (start 148.585 109.21) (end 151.765 106.03) (width 0.5) (layer "B.Cu") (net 3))
 (segment (start 151.765 106.03) (end 151.765 102.235) (width 0.5) (layer "B.Cu") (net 3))
 (segment (start 149.225 102.235) (end 149.225 104.76) (width 0.5) (layer "B.Cu") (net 4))
 (segment (start 149.225 104.76) (end 147.315 106.67) (width 0.5) (layer "B.Cu") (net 4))
 (segment (start 146.045 102.875) (end 146.685 102.235) (width 0.5) (layer "B.Cu") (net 5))
 (segment (start 146.045 109.21) (end 146.045 102.875) (width 0.5) (layer "B.Cu") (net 5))
 (segment (start 144.775 102.865) (end 144.775 106.67) (width 0.5) (layer "B.Cu") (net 6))
 (segment (start 144.145 102.235) (end 144.775 102.865) (width 0.5) (layer "B.Cu") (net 6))
 (segment (start 141.605 102.235) (end 143.505 104.135) (width 0.5) (layer "B.Cu") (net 7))
 (segment (start 143.505 104.135) (end 143.505 109.21) (width 0.5) (layer "B.Cu") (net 7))
 (segment (start 142.235 106.67) (end 139.065 103.5) (width 0.5) (layer "B.Cu") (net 8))
 (segment (start 139.065 103.5) (end 139.065 102.235) (width 0.5) (layer "B.Cu") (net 8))
 (segment (start 100.965 53.34) (end 104.475 53.34) (width 0.5) (layer "B.Cu") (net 9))
 (segment (start 104.475 55.88) (end 100.965 55.88) (width 0.5) (layer "B.Cu") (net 10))
 (segment (start 100.965 58.42) (end 104.475 58.42) (width 0.5) (layer "B.Cu") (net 11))
 (segment (start 104.475 60.96) (end 100.965 60.96) (width 0.5) (layer "B.Cu") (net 12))
 (segment (start 100.965 63.5) (end 104.475 63.5) (width 0.5) (layer "B.Cu") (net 13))
 (segment (start 104.475 66.04) (end 100.965 66.04) (width 0.5) (layer "B.Cu") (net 14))
 (segment (start 104.475 68.58) (end 100.965 68.58) (width 0.5) (layer "B.Cu") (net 15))
 (segment (start 100.965 71.12) (end 104.475 71.12) (width 0.5) (layer "B.Cu") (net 16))
 (segment (start 104.475 73.66) (end 100.965 73.66) (width 0.5) (layer "B.Cu") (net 17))
 (segment (start 100.965 76.2) (end 104.475 76.2) (width 0.5) (layer "B.Cu") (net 18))
 (segment (start 104.475 78.74) (end 100.965 78.74) (width 0.5) (layer "B.Cu") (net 19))
 (segment (start 100.965 81.28) (end 104.475 81.28) (width 0.5) (layer "B.Cu") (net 20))
 (segment (start 106.75 90.75) (end 106.75 104.62) (width 0.5) (layer "F.Cu") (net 22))
 (segment (start 106.75 104.62) (end 104.18 107.19) (width 0.5) (layer "F.Cu") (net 22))
 (segment (start 106.5 90.5) (end 106.75 90.75) (width 0.5) (layer "F.Cu") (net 22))
 (via (at 106.5 90.5) (size 1.2) (drill 0.6) (layers "F.Cu" "B.Cu") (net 22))
 (segment (start 104.475 88.9) (end 106.075 90.5) (width 0.5) (layer "B.Cu") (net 22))
 (segment (start 100.965 88.9) (end 104.475 88.9) (width 0.5) (layer "B.Cu") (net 22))
 (segment (start 106.075 90.5) (end 106.5 90.5) (width 0.5) (layer "B.Cu") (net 22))
 (segment (start 109 112.25) (end 105.94 112.25) (width 0.5) (layer "F.Cu") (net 23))
 (segment (start 109.75 94) (end 109.75 111.5) (width 0.5) (layer "F.Cu") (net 23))
 (segment (start 109.75 111.5) (end 109 112.25) (width 0.5) (layer "F.Cu") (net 23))
 (segment (start 105.94 112.25) (end 104.18 110.49) (width 0.5) (layer "F.Cu") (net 23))
 (segment (start 108 92.25) (end 109.75 94) (width 0.5) (layer "F.Cu") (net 23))
 (via (at 108 92.25) (size 1.2) (drill 0.6) (layers "F.Cu" "B.Cu") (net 23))
 (segment (start 108 92.25) (end 105.25 92.25) (width 0.5) (layer "B.Cu") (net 23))
 (segment (start 104.475 91.44) (end 100.965 91.44) (width 0.5) (layer "B.Cu") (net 23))
 (segment (start 104.475 91.475) (end 104.475 91.44) (width 0.5) (layer "B.Cu") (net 23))
 (segment (start 105.25 92.25) (end 104.475 91.475) (width 0.5) (layer "B.Cu") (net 23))
 (segment (start 104.475 96.52) (end 100.965 96.52) (width 0.5) (layer "B.Cu") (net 25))
 (segment (start 130.475 99.06) (end 133.985 99.06) (width 1) (layer "B.Cu") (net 46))
 (segment (start 133.985 96.52) (end 130.475 96.52) (width 0.5) (layer "B.Cu") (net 45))
 (segment (start 130.475 93.98) (end 133.985 93.98) (width 0.5) (layer "B.Cu") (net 44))
 (segment (start 133.985 91.44) (end 130.475 91.44) (width 0.5) (layer "B.Cu") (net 43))
 (segment (start 130.475 88.9) (end 133.985 88.9) (width 0.5) (layer "B.Cu") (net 42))
 (segment (start 133.985 86.36) (end 130.475 86.36) (width 0.5) (layer "B.Cu") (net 41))
 (segment (start 130.475 83.82) (end 133.985 83.82) (width 0.5) (layer "B.Cu") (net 40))
 (segment (start 133.985 78.74) (end 130.475 78.74) (width 0.5) (layer "B.Cu") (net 38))
 (segment (start 130.475 76.2) (end 133.985 76.2) (width 0.5) (layer "B.Cu") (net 37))
 (segment (start 133.985 73.66) (end 130.475 73.66) (width 0.5) (layer "B.Cu") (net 36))
 (segment (start 130.475 71.12) (end 133.985 71.12) (width 0.5) (layer "B.Cu") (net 35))
 (segment (start 133.985 68.58) (end 130.475 68.58) (width 0.5) (layer "B.Cu") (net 34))
 (segment (start 130.475 63.5) (end 133.985 63.5) (width 0.5) (layer "B.Cu") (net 33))
 (segment (start 133.985 60.96) (end 130.475 60.96) (width 0.5) (layer "B.Cu") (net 32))
 (segment (start 130.475 58.42) (end 133.985 58.42) (width 0.5) (layer "B.Cu") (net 31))
 (segment (start 133.985 55.88) (end 130.475 55.88) (width 0.5) (layer "B.Cu") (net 30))
 (segment (start 133.985 81.28) (end 130.475 81.28) (width 0.5) (layer "B.Cu") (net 39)))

